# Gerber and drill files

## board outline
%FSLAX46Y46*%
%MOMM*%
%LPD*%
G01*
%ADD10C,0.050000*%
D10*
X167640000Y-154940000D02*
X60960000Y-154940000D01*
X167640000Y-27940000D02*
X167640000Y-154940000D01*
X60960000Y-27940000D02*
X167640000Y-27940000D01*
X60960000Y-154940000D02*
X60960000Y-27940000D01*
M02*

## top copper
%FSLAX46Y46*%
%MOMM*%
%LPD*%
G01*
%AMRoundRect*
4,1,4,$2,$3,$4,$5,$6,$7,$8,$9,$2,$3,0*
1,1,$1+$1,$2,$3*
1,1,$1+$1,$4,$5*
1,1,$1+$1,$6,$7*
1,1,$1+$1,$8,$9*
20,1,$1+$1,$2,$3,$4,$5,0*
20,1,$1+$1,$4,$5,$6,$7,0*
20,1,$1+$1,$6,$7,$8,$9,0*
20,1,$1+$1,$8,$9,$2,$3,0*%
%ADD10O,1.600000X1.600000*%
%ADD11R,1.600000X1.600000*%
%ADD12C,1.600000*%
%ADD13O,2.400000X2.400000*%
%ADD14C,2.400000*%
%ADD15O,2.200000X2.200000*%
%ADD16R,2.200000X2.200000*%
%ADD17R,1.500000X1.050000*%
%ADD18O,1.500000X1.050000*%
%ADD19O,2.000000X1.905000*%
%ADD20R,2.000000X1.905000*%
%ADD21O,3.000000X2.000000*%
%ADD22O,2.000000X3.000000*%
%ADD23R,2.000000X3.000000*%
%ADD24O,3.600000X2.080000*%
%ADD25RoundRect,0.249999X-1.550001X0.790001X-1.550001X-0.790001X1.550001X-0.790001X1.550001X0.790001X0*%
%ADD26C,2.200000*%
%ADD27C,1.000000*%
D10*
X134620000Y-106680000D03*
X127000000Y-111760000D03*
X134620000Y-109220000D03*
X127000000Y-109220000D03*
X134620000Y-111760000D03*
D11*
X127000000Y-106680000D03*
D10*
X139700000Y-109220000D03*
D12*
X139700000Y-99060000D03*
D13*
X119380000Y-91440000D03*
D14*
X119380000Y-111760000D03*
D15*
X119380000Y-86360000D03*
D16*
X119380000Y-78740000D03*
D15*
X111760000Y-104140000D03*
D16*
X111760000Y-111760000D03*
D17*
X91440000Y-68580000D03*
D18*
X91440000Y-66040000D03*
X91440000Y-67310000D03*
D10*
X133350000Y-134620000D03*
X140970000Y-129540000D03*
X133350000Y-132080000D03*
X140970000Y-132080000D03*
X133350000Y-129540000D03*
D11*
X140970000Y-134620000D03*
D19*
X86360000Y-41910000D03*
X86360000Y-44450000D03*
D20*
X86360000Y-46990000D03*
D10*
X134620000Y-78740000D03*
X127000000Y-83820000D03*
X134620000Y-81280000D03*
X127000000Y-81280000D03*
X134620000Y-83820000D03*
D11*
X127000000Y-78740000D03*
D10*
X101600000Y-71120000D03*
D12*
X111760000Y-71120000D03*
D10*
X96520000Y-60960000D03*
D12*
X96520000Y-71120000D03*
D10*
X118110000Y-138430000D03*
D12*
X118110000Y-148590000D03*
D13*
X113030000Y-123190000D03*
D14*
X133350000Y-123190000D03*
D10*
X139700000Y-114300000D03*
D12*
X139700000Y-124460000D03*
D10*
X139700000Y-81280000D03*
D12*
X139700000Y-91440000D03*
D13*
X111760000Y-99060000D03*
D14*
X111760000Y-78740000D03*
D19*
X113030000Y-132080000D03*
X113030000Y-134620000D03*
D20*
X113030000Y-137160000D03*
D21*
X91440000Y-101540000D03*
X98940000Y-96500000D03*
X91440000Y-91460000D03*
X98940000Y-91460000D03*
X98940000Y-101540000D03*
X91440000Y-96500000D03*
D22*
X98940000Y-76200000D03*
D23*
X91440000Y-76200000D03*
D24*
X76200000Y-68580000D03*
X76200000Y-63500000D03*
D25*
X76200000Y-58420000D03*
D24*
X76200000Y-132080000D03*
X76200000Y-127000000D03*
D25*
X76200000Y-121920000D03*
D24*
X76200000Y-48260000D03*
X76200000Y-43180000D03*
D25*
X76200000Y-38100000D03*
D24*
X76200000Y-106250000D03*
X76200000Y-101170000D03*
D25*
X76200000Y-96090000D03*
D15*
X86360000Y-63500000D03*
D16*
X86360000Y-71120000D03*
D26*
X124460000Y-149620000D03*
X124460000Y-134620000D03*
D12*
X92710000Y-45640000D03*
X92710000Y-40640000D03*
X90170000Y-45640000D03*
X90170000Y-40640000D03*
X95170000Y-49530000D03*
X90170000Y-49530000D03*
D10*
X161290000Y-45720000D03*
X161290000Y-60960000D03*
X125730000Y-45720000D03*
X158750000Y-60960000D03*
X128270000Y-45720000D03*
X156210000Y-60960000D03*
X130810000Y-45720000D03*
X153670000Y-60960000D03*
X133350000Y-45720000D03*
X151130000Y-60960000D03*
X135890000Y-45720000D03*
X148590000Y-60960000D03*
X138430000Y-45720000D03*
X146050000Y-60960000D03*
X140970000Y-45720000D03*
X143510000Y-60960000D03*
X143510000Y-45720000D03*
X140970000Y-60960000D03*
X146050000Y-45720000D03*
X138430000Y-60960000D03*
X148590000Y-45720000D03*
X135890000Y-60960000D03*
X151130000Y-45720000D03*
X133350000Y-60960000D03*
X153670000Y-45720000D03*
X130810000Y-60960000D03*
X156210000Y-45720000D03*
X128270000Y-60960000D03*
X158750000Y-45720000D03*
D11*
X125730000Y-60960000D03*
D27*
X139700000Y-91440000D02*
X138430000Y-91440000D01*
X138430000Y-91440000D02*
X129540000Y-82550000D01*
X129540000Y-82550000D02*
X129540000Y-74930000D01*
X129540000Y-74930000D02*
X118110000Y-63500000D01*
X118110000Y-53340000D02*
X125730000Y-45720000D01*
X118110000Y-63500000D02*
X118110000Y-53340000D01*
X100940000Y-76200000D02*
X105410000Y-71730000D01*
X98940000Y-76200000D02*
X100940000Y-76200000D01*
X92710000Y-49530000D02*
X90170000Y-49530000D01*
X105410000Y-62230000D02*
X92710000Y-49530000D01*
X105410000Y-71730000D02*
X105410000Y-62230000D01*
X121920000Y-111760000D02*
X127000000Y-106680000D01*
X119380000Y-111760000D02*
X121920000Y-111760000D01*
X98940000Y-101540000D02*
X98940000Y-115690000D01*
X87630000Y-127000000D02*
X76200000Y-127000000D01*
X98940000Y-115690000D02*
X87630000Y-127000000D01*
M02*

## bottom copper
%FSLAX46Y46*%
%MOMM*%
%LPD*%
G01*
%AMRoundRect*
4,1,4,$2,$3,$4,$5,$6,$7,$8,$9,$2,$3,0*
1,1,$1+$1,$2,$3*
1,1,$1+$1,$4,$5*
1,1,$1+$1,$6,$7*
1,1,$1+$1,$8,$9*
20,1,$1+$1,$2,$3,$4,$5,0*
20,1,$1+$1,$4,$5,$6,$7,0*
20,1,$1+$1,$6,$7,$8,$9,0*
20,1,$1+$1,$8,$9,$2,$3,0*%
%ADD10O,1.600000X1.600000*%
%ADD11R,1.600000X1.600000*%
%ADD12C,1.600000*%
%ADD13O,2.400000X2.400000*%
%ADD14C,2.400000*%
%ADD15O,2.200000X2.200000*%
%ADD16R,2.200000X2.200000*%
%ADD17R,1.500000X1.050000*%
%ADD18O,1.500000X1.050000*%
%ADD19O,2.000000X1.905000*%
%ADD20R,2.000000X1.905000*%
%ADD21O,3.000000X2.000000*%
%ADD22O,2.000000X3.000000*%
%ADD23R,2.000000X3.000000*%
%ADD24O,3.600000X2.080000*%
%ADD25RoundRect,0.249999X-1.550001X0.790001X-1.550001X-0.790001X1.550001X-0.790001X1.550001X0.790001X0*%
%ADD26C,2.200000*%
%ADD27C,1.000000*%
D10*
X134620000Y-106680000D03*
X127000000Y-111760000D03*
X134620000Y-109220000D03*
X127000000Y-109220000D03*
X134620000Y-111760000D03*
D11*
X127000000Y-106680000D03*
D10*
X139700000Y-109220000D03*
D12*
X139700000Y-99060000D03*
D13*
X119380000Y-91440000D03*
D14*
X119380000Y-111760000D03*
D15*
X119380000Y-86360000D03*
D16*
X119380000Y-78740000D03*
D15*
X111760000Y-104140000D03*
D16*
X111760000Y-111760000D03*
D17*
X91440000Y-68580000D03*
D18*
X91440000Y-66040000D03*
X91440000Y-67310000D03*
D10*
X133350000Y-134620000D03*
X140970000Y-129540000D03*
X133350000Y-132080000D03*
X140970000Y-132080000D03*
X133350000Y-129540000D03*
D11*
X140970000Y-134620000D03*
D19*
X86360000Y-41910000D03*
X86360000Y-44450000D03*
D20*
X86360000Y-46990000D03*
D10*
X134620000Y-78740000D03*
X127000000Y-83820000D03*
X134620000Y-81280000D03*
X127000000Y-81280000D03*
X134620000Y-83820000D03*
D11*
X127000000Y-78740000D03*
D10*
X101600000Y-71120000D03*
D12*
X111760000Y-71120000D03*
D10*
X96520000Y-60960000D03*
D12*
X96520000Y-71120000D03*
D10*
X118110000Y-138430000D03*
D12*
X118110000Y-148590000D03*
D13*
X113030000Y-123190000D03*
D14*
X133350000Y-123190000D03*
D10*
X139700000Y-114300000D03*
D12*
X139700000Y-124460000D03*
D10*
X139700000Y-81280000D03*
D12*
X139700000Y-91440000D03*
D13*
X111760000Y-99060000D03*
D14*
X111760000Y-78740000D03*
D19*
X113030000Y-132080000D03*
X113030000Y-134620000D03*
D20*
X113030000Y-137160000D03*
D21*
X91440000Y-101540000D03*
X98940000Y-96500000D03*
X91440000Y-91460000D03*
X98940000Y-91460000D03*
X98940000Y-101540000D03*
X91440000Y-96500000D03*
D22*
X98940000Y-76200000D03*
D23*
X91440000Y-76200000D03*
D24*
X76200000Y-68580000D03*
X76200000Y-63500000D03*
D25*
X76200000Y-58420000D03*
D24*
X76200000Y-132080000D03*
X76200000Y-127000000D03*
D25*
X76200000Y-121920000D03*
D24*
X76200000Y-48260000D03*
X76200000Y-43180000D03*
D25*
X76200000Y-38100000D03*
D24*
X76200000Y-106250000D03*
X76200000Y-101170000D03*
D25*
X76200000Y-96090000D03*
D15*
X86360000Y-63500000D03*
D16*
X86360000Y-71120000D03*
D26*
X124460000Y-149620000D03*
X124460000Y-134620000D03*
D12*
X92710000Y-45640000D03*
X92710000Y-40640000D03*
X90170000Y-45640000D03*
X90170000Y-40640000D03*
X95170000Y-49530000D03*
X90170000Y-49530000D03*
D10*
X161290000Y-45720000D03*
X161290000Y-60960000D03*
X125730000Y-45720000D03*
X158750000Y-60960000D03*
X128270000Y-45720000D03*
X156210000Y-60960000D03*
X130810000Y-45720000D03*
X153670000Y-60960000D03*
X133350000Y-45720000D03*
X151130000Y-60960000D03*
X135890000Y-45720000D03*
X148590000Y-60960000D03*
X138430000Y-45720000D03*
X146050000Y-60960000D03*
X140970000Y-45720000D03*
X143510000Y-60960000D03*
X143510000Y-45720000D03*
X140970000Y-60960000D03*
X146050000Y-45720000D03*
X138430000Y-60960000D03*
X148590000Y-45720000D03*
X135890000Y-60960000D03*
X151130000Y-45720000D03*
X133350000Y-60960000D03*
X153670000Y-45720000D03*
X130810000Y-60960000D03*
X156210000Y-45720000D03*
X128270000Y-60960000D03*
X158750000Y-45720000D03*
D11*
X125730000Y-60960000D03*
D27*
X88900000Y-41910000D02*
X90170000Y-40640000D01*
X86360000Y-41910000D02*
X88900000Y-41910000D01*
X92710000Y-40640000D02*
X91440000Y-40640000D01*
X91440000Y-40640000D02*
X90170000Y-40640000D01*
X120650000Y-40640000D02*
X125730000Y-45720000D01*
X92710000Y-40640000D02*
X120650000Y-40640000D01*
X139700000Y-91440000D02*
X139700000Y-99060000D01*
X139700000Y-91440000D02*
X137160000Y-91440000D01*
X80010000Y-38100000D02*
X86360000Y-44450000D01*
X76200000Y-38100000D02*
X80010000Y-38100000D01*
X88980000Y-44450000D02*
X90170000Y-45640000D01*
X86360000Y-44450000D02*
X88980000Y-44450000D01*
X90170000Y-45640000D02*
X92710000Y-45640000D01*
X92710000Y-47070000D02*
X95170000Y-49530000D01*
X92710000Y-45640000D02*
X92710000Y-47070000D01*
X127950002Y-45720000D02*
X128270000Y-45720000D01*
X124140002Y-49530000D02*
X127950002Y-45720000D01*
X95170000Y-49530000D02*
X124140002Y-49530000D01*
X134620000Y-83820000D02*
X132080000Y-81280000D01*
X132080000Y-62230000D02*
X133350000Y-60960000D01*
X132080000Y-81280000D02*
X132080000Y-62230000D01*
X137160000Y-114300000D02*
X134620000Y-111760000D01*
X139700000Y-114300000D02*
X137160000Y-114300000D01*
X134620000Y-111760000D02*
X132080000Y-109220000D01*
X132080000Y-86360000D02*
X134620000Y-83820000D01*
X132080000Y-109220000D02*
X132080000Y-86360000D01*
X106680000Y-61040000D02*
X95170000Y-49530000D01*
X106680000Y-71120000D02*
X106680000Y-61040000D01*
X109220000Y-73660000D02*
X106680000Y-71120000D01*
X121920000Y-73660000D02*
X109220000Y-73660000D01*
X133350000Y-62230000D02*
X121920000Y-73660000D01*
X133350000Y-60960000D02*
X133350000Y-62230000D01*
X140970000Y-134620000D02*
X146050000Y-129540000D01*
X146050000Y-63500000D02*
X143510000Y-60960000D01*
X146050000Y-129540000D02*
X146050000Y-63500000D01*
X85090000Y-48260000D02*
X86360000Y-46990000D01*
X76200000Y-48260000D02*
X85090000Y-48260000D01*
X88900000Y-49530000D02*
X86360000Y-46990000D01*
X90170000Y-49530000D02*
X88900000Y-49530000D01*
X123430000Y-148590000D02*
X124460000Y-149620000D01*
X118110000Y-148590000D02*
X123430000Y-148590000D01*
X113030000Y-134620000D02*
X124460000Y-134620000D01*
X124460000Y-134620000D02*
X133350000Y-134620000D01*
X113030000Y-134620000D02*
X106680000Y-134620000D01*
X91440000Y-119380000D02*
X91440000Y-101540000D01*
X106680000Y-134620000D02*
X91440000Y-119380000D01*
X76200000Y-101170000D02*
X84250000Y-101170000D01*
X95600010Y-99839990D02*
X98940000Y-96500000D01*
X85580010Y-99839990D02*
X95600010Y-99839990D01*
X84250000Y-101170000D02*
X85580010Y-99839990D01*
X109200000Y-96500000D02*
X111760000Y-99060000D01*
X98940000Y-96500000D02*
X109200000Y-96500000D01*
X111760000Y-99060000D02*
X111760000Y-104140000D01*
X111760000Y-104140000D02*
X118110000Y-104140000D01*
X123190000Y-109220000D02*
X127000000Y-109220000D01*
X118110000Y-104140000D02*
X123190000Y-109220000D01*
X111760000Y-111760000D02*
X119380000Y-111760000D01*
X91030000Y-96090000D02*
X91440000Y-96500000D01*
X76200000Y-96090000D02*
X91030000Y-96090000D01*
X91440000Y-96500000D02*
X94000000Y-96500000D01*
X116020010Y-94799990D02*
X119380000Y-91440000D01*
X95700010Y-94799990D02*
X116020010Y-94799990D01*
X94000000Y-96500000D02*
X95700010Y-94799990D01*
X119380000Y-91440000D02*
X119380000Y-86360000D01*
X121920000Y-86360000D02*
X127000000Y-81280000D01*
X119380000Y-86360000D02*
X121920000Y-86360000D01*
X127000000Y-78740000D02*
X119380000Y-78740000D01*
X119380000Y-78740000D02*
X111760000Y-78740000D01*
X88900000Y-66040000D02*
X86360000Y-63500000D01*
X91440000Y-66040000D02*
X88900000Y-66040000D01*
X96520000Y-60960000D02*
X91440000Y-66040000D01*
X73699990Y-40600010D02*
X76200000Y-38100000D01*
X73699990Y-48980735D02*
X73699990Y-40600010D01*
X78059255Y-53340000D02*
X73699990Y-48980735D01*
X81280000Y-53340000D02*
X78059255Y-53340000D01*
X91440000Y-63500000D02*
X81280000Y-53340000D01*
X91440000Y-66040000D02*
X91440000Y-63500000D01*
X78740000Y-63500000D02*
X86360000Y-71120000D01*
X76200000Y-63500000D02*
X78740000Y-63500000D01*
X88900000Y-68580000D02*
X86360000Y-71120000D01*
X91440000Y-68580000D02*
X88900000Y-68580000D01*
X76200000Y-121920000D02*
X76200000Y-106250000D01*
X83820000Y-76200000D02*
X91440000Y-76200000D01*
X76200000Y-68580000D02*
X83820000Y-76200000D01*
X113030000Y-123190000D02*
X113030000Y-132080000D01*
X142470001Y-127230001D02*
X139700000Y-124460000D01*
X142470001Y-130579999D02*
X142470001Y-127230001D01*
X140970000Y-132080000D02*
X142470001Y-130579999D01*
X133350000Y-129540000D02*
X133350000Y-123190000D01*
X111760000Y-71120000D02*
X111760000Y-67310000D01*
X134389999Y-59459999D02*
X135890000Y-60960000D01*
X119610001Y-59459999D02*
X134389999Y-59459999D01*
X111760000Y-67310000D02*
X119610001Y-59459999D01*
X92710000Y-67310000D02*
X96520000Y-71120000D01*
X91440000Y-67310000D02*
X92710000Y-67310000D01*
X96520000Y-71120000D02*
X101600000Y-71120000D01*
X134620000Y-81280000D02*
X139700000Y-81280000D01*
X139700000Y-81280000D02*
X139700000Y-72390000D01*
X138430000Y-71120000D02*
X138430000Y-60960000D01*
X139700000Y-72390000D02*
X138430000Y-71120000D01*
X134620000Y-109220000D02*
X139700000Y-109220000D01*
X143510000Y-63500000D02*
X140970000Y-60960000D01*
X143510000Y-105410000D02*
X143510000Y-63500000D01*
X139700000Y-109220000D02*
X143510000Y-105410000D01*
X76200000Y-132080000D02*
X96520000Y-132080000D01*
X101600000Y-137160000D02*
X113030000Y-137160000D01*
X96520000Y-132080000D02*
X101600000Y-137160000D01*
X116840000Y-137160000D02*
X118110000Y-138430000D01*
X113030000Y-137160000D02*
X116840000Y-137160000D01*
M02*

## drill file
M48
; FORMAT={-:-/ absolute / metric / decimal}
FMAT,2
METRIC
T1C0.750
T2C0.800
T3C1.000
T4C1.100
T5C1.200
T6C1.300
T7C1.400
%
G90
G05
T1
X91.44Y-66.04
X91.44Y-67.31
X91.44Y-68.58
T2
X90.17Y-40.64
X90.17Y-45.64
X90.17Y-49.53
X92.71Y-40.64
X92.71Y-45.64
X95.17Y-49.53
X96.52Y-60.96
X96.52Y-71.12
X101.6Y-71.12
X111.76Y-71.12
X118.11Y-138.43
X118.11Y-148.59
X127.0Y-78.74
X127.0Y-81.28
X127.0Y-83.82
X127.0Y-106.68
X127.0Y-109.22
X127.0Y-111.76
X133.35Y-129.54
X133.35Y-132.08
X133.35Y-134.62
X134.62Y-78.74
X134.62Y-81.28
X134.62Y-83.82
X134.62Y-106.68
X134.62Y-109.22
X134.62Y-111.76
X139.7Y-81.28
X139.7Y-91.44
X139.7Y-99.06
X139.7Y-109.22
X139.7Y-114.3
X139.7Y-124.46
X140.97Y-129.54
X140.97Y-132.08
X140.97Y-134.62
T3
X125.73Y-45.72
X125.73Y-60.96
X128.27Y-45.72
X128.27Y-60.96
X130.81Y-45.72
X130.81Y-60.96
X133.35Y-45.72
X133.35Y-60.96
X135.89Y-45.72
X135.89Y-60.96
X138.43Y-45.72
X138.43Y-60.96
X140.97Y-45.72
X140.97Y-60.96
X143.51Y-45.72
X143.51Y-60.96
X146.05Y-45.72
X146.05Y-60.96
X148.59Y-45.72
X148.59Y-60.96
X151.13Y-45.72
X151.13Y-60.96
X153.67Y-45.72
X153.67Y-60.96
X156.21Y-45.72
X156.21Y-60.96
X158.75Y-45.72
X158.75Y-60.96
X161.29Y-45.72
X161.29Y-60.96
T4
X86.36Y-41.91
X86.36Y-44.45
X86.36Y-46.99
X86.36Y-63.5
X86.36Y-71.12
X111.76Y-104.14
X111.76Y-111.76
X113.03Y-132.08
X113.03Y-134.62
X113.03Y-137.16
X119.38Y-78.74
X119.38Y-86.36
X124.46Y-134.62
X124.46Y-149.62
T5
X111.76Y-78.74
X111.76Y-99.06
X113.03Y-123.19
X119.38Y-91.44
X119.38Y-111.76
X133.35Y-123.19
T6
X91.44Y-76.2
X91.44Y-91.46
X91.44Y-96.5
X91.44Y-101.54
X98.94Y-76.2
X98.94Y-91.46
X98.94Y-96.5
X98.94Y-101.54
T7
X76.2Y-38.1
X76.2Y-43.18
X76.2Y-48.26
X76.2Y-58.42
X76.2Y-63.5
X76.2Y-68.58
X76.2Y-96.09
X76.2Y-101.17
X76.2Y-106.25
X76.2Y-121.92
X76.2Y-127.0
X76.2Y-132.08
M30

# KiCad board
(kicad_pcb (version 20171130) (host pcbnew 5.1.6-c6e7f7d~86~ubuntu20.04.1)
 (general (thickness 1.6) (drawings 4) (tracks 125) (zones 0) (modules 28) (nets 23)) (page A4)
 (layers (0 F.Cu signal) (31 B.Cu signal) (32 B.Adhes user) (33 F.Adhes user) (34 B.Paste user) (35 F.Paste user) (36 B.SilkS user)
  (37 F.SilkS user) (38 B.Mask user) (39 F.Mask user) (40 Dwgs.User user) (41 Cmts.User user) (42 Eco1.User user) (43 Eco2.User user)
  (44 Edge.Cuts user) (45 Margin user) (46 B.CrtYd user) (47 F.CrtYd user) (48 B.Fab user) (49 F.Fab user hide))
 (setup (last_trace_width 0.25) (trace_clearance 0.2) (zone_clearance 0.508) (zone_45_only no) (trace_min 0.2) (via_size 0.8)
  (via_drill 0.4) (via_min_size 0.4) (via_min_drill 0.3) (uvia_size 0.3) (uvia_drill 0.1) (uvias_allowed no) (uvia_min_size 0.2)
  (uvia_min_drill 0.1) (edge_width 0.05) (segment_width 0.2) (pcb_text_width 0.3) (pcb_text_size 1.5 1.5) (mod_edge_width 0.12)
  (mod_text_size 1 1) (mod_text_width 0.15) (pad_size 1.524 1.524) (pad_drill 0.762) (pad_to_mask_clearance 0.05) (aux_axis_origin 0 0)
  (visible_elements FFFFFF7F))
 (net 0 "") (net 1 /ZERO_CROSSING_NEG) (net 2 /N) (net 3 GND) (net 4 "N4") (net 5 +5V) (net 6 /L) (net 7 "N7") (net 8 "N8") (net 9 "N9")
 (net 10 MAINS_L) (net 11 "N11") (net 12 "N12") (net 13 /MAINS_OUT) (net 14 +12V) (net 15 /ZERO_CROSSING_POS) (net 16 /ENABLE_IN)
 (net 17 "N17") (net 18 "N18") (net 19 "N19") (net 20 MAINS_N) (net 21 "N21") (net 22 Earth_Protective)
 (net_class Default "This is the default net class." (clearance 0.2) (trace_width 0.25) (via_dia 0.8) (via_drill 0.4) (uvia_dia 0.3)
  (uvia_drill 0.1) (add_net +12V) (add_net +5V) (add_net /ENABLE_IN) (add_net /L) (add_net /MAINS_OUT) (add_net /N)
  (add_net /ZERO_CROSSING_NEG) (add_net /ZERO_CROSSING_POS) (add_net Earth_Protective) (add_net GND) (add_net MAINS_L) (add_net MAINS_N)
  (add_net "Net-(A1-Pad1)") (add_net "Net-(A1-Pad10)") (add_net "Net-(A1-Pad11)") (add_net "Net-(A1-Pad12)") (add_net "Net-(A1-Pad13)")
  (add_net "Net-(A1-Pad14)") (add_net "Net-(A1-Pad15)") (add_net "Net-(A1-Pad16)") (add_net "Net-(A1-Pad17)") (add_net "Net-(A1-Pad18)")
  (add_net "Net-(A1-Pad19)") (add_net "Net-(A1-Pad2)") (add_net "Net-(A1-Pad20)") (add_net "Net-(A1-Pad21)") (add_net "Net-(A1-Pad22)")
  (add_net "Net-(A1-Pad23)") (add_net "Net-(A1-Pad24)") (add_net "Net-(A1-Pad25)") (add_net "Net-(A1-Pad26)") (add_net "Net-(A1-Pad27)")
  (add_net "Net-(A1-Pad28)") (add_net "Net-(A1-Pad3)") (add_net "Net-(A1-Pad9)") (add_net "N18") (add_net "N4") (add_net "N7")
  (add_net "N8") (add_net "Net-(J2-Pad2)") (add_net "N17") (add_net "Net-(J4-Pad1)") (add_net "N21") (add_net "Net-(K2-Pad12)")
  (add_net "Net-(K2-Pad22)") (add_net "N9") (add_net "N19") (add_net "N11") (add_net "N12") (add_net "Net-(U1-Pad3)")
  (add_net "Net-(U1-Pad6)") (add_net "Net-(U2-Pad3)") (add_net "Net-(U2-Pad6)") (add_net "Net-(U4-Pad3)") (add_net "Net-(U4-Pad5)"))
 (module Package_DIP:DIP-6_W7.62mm (layer F.Cu) (at 127 106.68)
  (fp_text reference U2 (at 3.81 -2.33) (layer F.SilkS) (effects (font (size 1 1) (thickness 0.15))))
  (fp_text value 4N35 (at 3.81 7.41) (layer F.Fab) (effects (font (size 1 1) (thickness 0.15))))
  (pad 6 thru_hole oval (at 7.62 0) (size 1.6 1.6) (drill 0.8) (layers *.Cu *.Mask))
  (pad 3 thru_hole oval (at 0 5.08) (size 1.6 1.6) (drill 0.8) (layers *.Cu *.Mask))
  (pad 5 thru_hole oval (at 7.62 2.54) (size 1.6 1.6) (drill 0.8) (layers *.Cu *.Mask) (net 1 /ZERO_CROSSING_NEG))
  (pad 2 thru_hole oval (at 0 2.54) (size 1.6 1.6) (drill 0.8) (layers *.Cu *.Mask) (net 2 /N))
  (pad 4 thru_hole oval (at 7.62 5.08) (size 1.6 1.6) (drill 0.8) (layers *.Cu *.Mask) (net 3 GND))
  (pad 1 thru_hole rect (at 0 0) (size 1.6 1.6) (drill 0.8) (layers *.Cu *.Mask) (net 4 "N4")))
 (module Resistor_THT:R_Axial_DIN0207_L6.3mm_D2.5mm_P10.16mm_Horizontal (layer F.Cu) (at 139.7 99.06 270)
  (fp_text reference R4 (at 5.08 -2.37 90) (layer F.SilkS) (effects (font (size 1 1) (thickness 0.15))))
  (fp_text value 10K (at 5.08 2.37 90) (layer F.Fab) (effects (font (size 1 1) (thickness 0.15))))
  (pad 2 thru_hole oval (at 10.16 0 270) (size 1.6 1.6) (drill 0.8) (layers *.Cu *.Mask) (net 1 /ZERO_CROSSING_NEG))
  (pad 1 thru_hole circle (at 0 0 270) (size 1.6 1.6) (drill 0.8) (layers *.Cu *.Mask) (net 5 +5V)))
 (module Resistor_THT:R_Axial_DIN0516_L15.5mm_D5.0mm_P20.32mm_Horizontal (layer F.Cu) (at 119.38 111.76 90)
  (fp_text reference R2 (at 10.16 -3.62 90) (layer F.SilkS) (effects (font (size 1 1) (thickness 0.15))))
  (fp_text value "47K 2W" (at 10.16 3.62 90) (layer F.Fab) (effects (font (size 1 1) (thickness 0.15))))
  (pad 2 thru_hole oval (at 20.32 0 90) (size 2.4 2.4) (drill 1.2) (layers *.Cu *.Mask) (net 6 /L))
  (pad 1 thru_hole circle (at 0 0 90) (size 2.4 2.4) (drill 1.2) (layers *.Cu *.Mask) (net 4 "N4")))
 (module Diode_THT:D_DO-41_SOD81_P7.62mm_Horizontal (layer F.Cu) (at 119.38 78.74 270)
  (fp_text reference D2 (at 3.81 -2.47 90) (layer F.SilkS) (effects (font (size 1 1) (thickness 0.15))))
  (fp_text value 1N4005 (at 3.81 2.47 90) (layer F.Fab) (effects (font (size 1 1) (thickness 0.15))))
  (pad 2 thru_hole oval (at 7.62 0 270) (size 2.2 2.2) (drill 1.1) (layers *.Cu *.Mask) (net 6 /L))
  (pad 1 thru_hole rect (at 0 0 270) (size 2.2 2.2) (drill 1.1) (layers *.Cu *.Mask) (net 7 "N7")))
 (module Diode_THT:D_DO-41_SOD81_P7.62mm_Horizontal (layer F.Cu) (at 111.76 111.76 90)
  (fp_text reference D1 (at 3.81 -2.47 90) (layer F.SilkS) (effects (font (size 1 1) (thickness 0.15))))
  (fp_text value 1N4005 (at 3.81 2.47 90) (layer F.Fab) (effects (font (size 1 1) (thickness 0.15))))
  (pad 2 thru_hole oval (at 7.62 0 90) (size 2.2 2.2) (drill 1.1) (layers *.Cu *.Mask) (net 2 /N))
  (pad 1 thru_hole rect (at 0 0 90) (size 2.2 2.2) (drill 1.1) (layers *.Cu *.Mask) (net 4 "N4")))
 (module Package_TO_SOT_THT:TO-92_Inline (layer F.Cu) (at 91.44 68.58 90)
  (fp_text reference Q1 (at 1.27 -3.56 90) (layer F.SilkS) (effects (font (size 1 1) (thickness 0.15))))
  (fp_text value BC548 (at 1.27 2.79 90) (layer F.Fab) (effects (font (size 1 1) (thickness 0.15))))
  (pad 1 thru_hole rect (at 0 0 90) (size 1.05 1.5) (drill 0.75) (layers *.Cu *.Mask) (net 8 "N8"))
  (pad 3 thru_hole oval (at 2.54 0 90) (size 1.05 1.5) (drill 0.75) (layers *.Cu *.Mask) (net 3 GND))
  (pad 2 thru_hole oval (at 1.27 0 90) (size 1.05 1.5) (drill 0.75) (layers *.Cu *.Mask) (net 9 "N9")))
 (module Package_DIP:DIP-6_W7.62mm (layer F.Cu) (at 140.97 134.62 180)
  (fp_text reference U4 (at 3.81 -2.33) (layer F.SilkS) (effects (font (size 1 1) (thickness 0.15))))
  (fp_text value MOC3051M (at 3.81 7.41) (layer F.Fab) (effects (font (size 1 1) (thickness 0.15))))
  (pad 6 thru_hole oval (at 7.62 0 180) (size 1.6 1.6) (drill 0.8) (layers *.Cu *.Mask) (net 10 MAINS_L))
  (pad 3 thru_hole oval (at 0 5.08 180) (size 1.6 1.6) (drill 0.8) (layers *.Cu *.Mask))
  (pad 5 thru_hole oval (at 7.62 2.54 180) (size 1.6 1.6) (drill 0.8) (layers *.Cu *.Mask))
  (pad 2 thru_hole oval (at 0 2.54 180) (size 1.6 1.6) (drill 0.8) (layers *.Cu *.Mask) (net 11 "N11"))
  (pad 4 thru_hole oval (at 7.62 5.08 180) (size 1.6 1.6) (drill 0.8) (layers *.Cu *.Mask) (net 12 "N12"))
  (pad 1 thru_hole rect (at 0 0 180) (size 1.6 1.6) (drill 0.8) (layers *.Cu *.Mask) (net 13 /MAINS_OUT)))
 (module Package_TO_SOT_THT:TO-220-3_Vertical (layer F.Cu) (at 86.36 46.99 90)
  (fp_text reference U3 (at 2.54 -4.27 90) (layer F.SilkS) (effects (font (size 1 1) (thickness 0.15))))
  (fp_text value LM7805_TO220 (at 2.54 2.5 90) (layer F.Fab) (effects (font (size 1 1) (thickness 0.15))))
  (pad 3 thru_hole oval (at 5.08 0 90) (size 1.905 2) (drill 1.1) (layers *.Cu *.Mask) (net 5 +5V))
  (pad 2 thru_hole oval (at 2.54 0 90) (size 1.905 2) (drill 1.1) (layers *.Cu *.Mask) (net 3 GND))
  (pad 1 thru_hole rect (at 0 0 90) (size 1.905 2) (drill 1.1) (layers *.Cu *.Mask) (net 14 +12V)))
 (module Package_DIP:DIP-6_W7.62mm (layer F.Cu) (at 127 78.74)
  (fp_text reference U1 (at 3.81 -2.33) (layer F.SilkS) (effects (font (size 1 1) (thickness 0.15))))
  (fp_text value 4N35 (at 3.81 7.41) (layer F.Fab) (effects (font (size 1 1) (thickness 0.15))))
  (pad 6 thru_hole oval (at 7.62 0) (size 1.6 1.6) (drill 0.8) (layers *.Cu *.Mask))
  (pad 3 thru_hole oval (at 0 5.08) (size 1.6 1.6) (drill 0.8) (layers *.Cu *.Mask))
  (pad 5 thru_hole oval (at 7.62 2.54) (size 1.6 1.6) (drill 0.8) (layers *.Cu *.Mask) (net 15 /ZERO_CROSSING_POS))
  (pad 2 thru_hole oval (at 0 2.54) (size 1.6 1.6) (drill 0.8) (layers *.Cu *.Mask) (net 6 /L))
  (pad 4 thru_hole oval (at 7.62 5.08) (size 1.6 1.6) (drill 0.8) (layers *.Cu *.Mask) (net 3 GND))
  (pad 1 thru_hole rect (at 0 0) (size 1.6 1.6) (drill 0.8) (layers *.Cu *.Mask) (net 7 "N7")))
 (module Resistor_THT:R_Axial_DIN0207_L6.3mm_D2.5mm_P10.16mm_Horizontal (layer F.Cu) (at 111.76 71.12 180)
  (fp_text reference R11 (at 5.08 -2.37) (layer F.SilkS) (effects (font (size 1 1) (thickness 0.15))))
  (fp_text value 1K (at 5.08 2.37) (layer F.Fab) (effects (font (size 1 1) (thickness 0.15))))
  (pad 2 thru_hole oval (at 10.16 0 180) (size 1.6 1.6) (drill 0.8) (layers *.Cu *.Mask) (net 9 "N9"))
  (pad 1 thru_hole circle (at 0 0 180) (size 1.6 1.6) (drill 0.8) (layers *.Cu *.Mask) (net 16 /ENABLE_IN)))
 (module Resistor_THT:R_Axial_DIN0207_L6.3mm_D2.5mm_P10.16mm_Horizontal (layer F.Cu) (at 96.52 71.12 90)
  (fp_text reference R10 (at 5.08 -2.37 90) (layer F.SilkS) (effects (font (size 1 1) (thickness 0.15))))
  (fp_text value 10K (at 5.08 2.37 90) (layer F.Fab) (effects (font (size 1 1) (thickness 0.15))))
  (pad 2 thru_hole oval (at 10.16 0 90) (size 1.6 1.6) (drill 0.8) (layers *.Cu *.Mask) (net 3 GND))
  (pad 1 thru_hole circle (at 0 0 90) (size 1.6 1.6) (drill 0.8) (layers *.Cu *.Mask) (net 9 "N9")))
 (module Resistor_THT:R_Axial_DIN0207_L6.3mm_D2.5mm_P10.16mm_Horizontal (layer F.Cu) (at 118.11 148.59 90)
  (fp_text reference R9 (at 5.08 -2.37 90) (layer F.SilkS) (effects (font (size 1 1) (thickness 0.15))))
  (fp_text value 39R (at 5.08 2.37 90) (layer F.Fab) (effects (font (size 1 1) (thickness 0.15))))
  (pad 2 thru_hole oval (at 10.16 0 90) (size 1.6 1.6) (drill 0.8) (layers *.Cu *.Mask) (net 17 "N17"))
  (pad 1 thru_hole circle (at 0 0 90) (size 1.6 1.6) (drill 0.8) (layers *.Cu *.Mask) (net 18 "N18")))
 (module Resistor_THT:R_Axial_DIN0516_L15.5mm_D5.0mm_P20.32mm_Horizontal (layer F.Cu) (at 133.35 123.19 180)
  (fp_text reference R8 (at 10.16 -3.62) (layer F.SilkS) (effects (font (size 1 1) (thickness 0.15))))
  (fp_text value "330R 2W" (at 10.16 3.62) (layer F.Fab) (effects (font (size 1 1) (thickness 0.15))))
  (pad 2 thru_hole oval (at 20.32 0 180) (size 2.4 2.4) (drill 1.2) (layers *.Cu *.Mask) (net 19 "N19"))
  (pad 1 thru_hole circle (at 0 0 180) (size 2.4 2.4) (drill 1.2) (layers *.Cu *.Mask) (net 12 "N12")))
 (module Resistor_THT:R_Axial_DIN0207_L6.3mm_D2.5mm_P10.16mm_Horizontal (layer F.Cu) (at 139.7 124.46 90)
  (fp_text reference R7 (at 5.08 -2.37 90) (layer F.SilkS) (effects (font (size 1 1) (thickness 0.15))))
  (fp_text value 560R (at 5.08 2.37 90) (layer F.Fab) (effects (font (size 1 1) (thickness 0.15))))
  (pad 2 thru_hole oval (at 10.16 0 90) (size 1.6 1.6) (drill 0.8) (layers *.Cu *.Mask) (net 3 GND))
  (pad 1 thru_hole circle (at 0 0 90) (size 1.6 1.6) (drill 0.8) (layers *.Cu *.Mask) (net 11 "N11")))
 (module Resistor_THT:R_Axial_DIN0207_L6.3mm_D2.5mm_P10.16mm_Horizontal (layer F.Cu) (at 139.7 91.44 90)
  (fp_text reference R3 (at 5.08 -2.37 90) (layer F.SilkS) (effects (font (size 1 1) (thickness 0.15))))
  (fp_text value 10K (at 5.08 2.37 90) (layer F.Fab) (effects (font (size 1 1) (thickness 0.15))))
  (pad 2 thru_hole oval (at 10.16 0 90) (size 1.6 1.6) (drill 0.8) (layers *.Cu *.Mask) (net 15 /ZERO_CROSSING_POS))
  (pad 1 thru_hole circle (at 0 0 90) (size 1.6 1.6) (drill 0.8) (layers *.Cu *.Mask) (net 5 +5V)))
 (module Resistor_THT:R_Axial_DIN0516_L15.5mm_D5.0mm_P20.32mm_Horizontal (layer F.Cu) (at 111.76 78.74 270)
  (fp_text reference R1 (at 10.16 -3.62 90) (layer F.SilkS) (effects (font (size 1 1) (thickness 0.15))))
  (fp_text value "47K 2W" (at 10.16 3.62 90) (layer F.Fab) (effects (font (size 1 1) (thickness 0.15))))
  (pad 2 thru_hole oval (at 20.32 0 270) (size 2.4 2.4) (drill 1.2) (layers *.Cu *.Mask) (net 2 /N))
  (pad 1 thru_hole circle (at 0 0 270) (size 2.4 2.4) (drill 1.2) (layers *.Cu *.Mask) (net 7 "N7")))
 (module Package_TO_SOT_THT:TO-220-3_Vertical (layer F.Cu) (at 113.03 137.16 90)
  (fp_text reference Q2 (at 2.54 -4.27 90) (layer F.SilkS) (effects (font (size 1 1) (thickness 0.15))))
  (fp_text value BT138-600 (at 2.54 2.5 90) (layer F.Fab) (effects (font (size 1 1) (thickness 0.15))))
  (pad 3 thru_hole oval (at 5.08 0 90) (size 1.905 2) (drill 1.1) (layers *.Cu *.Mask) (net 19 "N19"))
  (pad 2 thru_hole oval (at 2.54 0 90) (size 1.905 2) (drill 1.1) (layers *.Cu *.Mask) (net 10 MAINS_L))
  (pad 1 thru_hole rect (at 0 0 90) (size 1.905 2) (drill 1.1) (layers *.Cu *.Mask) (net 17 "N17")))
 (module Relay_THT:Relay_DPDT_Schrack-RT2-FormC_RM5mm (layer F.Cu) (at 91.44 76.2 270)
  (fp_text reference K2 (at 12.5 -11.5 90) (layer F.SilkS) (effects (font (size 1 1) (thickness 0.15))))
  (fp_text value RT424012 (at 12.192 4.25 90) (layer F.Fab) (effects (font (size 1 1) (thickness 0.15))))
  (pad 14 thru_hole oval (at 25.34 0 90) (size 2 3) (drill 1.3) (layers *.Cu *.Mask) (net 10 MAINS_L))
  (pad 21 thru_hole oval (at 20.3 -7.5 90) (size 2 3) (drill 1.3) (layers *.Cu *.Mask) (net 2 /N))
  (pad 12 thru_hole oval (at 15.26 0 90) (size 2 3) (drill 1.3) (layers *.Cu *.Mask))
  (pad 22 thru_hole oval (at 15.26 -7.5 90) (size 2 3) (drill 1.3) (layers *.Cu *.Mask))
  (pad 24 thru_hole oval (at 25.34 -7.5 90) (size 2 3) (drill 1.3) (layers *.Cu *.Mask) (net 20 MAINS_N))
  (pad 11 thru_hole oval (at 20.3 0 90) (size 2 3) (drill 1.3) (layers *.Cu *.Mask) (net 6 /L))
  (pad A2 thru_hole oval (at 0 -7.5 90) (size 3 2) (drill 1.3) (layers *.Cu *.Mask) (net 14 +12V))
  (pad A1 thru_hole rect (at 0 0 90) (size 3 2) (drill 1.3) (layers *.Cu *.Mask) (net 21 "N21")))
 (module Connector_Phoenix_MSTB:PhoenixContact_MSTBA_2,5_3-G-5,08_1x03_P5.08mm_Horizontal (layer F.Cu) (at 76.2 58.42 270)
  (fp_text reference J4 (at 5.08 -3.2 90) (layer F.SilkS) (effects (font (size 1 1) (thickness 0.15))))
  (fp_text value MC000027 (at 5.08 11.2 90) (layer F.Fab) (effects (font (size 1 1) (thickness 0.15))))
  (pad 3 thru_hole oval (at 10.16 0 270) (size 2.08 3.6) (drill 1.4) (layers *.Cu *.Mask) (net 21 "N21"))
  (pad 2 thru_hole oval (at 5.08 0 270) (size 2.08 3.6) (drill 1.4) (layers *.Cu *.Mask) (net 8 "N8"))
  (pad 1 thru_hole roundrect (at 0 0 270) (size 2.08 3.6) (drill 1.4) (layers *.Cu *.Mask) (roundrect_rratio 0.120192)))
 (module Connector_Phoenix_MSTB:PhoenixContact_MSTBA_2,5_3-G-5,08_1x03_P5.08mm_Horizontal (layer F.Cu) (at 76.2 121.92 270)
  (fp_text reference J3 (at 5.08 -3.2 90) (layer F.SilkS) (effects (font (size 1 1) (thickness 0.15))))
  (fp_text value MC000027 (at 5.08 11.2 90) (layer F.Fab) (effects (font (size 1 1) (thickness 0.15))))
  (pad 3 thru_hole oval (at 10.16 0 270) (size 2.08 3.6) (drill 1.4) (layers *.Cu *.Mask) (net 17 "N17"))
  (pad 2 thru_hole oval (at 5.08 0 270) (size 2.08 3.6) (drill 1.4) (layers *.Cu *.Mask) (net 20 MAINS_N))
  (pad 1 thru_hole roundrect (at 0 0 270) (size 2.08 3.6) (drill 1.4) (layers *.Cu *.Mask) (roundrect_rratio 0.120192)
   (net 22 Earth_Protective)))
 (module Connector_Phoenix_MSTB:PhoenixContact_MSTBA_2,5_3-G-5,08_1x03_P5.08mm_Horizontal (layer F.Cu) (at 76.2 38.1 270)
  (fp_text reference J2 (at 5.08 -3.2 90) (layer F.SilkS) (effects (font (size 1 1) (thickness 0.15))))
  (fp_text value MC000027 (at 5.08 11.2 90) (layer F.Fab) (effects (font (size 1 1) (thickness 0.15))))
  (pad 3 thru_hole oval (at 10.16 0 270) (size 2.08 3.6) (drill 1.4) (layers *.Cu *.Mask) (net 14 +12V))
  (pad 2 thru_hole oval (at 5.08 0 270) (size 2.08 3.6) (drill 1.4) (layers *.Cu *.Mask))
  (pad 1 thru_hole roundrect (at 0 0 270) (size 2.08 3.6) (drill 1.4) (layers *.Cu *.Mask) (roundrect_rratio 0.120192) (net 3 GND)))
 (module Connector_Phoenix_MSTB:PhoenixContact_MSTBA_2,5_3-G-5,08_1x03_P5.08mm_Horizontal (layer F.Cu) (at 76.2 96.09 270)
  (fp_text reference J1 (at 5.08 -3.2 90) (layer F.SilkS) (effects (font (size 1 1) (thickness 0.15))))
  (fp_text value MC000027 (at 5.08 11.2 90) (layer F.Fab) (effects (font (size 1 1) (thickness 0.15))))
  (pad 3 thru_hole oval (at 10.16 0 270) (size 2.08 3.6) (drill 1.4) (layers *.Cu *.Mask) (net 22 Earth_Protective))
  (pad 2 thru_hole oval (at 5.08 0 270) (size 2.08 3.6) (drill 1.4) (layers *.Cu *.Mask) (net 2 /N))
  (pad 1 thru_hole roundrect (at 0 0 270) (size 2.08 3.6) (drill 1.4) (layers *.Cu *.Mask) (roundrect_rratio 0.120192) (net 6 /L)))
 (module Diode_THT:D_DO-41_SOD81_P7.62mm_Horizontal (layer F.Cu) (at 86.36 71.12 90)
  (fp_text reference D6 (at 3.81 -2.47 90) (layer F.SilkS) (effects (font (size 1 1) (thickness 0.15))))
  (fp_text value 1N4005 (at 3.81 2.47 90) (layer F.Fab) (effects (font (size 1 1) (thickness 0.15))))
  (pad 2 thru_hole oval (at 7.62 0 90) (size 2.2 2.2) (drill 1.1) (layers *.Cu *.Mask) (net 3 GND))
  (pad 1 thru_hole rect (at 0 0 90) (size 2.2 2.2) (drill 1.1) (layers *.Cu *.Mask) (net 8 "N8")))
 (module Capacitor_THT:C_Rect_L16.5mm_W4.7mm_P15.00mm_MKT (layer F.Cu) (at 124.46 134.62 270)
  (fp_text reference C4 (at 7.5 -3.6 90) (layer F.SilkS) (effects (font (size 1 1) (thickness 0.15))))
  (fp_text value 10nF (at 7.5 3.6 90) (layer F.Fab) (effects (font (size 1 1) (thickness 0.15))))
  (pad 2 thru_hole circle (at 15 0 270) (size 2.2 2.2) (drill 1.1) (layers *.Cu *.Mask) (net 18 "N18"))
  (pad 1 thru_hole circle (at 0 0 270) (size 2.2 2.2) (drill 1.1) (layers *.Cu *.Mask) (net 10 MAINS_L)))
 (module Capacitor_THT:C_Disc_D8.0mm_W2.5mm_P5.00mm (layer F.Cu) (at 92.71 40.64 270)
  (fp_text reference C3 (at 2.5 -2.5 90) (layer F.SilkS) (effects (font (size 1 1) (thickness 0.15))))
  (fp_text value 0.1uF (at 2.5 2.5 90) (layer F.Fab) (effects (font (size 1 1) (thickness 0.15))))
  (pad 2 thru_hole circle (at 5 0 270) (size 1.6 1.6) (drill 0.8) (layers *.Cu *.Mask) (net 3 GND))
  (pad 1 thru_hole circle (at 0 0 270) (size 1.6 1.6) (drill 0.8) (layers *.Cu *.Mask) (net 5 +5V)))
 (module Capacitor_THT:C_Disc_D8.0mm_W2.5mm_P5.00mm (layer F.Cu) (at 90.17 40.64 270)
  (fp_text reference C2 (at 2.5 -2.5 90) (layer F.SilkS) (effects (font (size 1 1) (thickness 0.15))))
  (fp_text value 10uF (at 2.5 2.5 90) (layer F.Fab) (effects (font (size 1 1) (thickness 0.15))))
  (pad 2 thru_hole circle (at 5 0 270) (size 1.6 1.6) (drill 0.8) (layers *.Cu *.Mask) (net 3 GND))
  (pad 1 thru_hole circle (at 0 0 270) (size 1.6 1.6) (drill 0.8) (layers *.Cu *.Mask) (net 5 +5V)))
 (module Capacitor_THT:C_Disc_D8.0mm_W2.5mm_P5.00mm (layer F.Cu) (at 90.17 49.53)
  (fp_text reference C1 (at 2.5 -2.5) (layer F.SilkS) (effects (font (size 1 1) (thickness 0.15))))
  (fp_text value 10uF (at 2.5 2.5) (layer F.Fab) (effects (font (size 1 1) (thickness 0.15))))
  (pad 2 thru_hole circle (at 5 0) (size 1.6 1.6) (drill 0.8) (layers *.Cu *.Mask) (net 3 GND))
  (pad 1 thru_hole circle (at 0 0) (size 1.6 1.6) (drill 0.8) (layers *.Cu *.Mask) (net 14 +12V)))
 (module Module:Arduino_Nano (layer F.Cu) (at 125.73 60.96 90)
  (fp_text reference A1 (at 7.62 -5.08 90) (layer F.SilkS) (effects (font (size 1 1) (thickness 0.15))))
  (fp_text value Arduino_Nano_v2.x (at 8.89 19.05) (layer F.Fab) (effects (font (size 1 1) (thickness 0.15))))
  (pad 16 thru_hole oval (at 15.24 35.56 90) (size 1.6 1.6) (drill 1) (layers *.Cu *.Mask))
  (pad 15 thru_hole oval (at 0 35.56 90) (size 1.6 1.6) (drill 1) (layers *.Cu *.Mask))
  (pad 30 thru_hole oval (at 15.24 0 90) (size 1.6 1.6) (drill 1) (layers *.Cu *.Mask) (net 5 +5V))
  (pad 14 thru_hole oval (at 0 33.02 90) (size 1.6 1.6) (drill 1) (layers *.Cu *.Mask))
  (pad 29 thru_hole oval (at 15.24 2.54 90) (size 1.6 1.6) (drill 1) (layers *.Cu *.Mask) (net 3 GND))
  (pad 13 thru_hole oval (at 0 30.48 90) (size 1.6 1.6) (drill 1) (layers *.Cu *.Mask))
  (pad 28 thru_hole oval (at 15.24 5.08 90) (size 1.6 1.6) (drill 1) (layers *.Cu *.Mask))
  (pad 12 thru_hole oval (at 0 27.94 90) (size 1.6 1.6) (drill 1) (layers *.Cu *.Mask))
  (pad 27 thru_hole oval (at 15.24 7.62 90) (size 1.6 1.6) (drill 1) (layers *.Cu *.Mask))
  (pad 11 thru_hole oval (at 0 25.4 90) (size 1.6 1.6) (drill 1) (layers *.Cu *.Mask))
  (pad 26 thru_hole oval (at 15.24 10.16 90) (size 1.6 1.6) (drill 1) (layers *.Cu *.Mask))
  (pad 10 thru_hole oval (at 0 22.86 90) (size 1.6 1.6) (drill 1) (layers *.Cu *.Mask))
  (pad 25 thru_hole oval (at 15.24 12.7 90) (size 1.6 1.6) (drill 1) (layers *.Cu *.Mask))
  (pad 9 thru_hole oval (at 0 20.32 90) (size 1.6 1.6) (drill 1) (layers *.Cu *.Mask))
  (pad 24 thru_hole oval (at 15.24 15.24 90) (size 1.6 1.6) (drill 1) (layers *.Cu *.Mask))
  (pad 8 thru_hole oval (at 0 17.78 90) (size 1.6 1.6) (drill 1) (layers *.Cu *.Mask) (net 13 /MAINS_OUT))
  (pad 23 thru_hole oval (at 15.24 17.78 90) (size 1.6 1.6) (drill 1) (layers *.Cu *.Mask))
  (pad 7 thru_hole oval (at 0 15.24 90) (size 1.6 1.6) (drill 1) (layers *.Cu *.Mask) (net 1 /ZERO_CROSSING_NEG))
  (pad 22 thru_hole oval (at 15.24 20.32 90) (size 1.6 1.6) (drill 1) (layers *.Cu *.Mask))
  (pad 6 thru_hole oval (at 0 12.7 90) (size 1.6 1.6) (drill 1) (layers *.Cu *.Mask) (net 15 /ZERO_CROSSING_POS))
  (pad 21 thru_hole oval (at 15.24 22.86 90) (size 1.6 1.6) (drill 1) (layers *.Cu *.Mask))
  (pad 5 thru_hole oval (at 0 10.16 90) (size 1.6 1.6) (drill 1) (layers *.Cu *.Mask) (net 16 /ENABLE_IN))
  (pad 20 thru_hole oval (at 15.24 25.4 90) (size 1.6 1.6) (drill 1) (layers *.Cu *.Mask))
  (pad 4 thru_hole oval (at 0 7.62 90) (size 1.6 1.6) (drill 1) (layers *.Cu *.Mask) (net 3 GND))
  (pad 19 thru_hole oval (at 15.24 27.94 90) (size 1.6 1.6) (drill 1) (layers *.Cu *.Mask))
  (pad 3 thru_hole oval (at 0 5.08 90) (size 1.6 1.6) (drill 1) (layers *.Cu *.Mask))
  (pad 18 thru_hole oval (at 15.24 30.48 90) (size 1.6 1.6) (drill 1) (layers *.Cu *.Mask))
  (pad 2 thru_hole oval (at 0 2.54 90) (size 1.6 1.6) (drill 1) (layers *.Cu *.Mask))
  (pad 17 thru_hole oval (at 15.24 33.02 90) (size 1.6 1.6) (drill 1) (layers *.Cu *.Mask))
  (pad 1 thru_hole rect (at 0 0 90) (size 1.6 1.6) (drill 1) (layers *.Cu *.Mask)))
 (gr_line (start 167.64 154.94) (end 60.96 154.94) (layer Edge.Cuts) (width 0.05))
 (gr_line (start 167.64 27.94) (end 167.64 154.94) (layer Edge.Cuts) (width 0.05))
 (gr_line (start 60.96 27.94) (end 167.64 27.94) (layer Edge.Cuts) (width 0.05))
 (gr_line (start 60.96 154.94) (end 60.96 27.94) (layer Edge.Cuts) (width 0.05))
 (segment (start 88.9 41.91) (end 90.17 40.64) (width 1) (layer B.Cu) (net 5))
 (segment (start 86.36 41.91) (end 88.9 41.91) (width 1) (layer B.Cu) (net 5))
 (segment (start 92.71 40.64) (end 91.44 40.64) (width 1) (layer B.Cu) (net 5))
 (segment (start 91.44 40.64) (end 90.17 40.64) (width 1) (layer B.Cu) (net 5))
 (segment (start 120.65 40.64) (end 125.73 45.72) (width 1) (layer B.Cu) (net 5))
 (segment (start 92.71 40.64) (end 120.65 40.64) (width 1) (layer B.Cu) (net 5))
 (segment (start 139.7 91.44) (end 139.7 99.06) (width 1) (layer B.Cu) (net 5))
 (segment (start 139.7 91.44) (end 137.16 91.44) (width 1) (layer B.Cu) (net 5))
 (segment (start 139.7 91.44) (end 138.43 91.44) (width 1) (layer F.Cu) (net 5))
 (segment (start 138.43 91.44) (end 129.54 82.55) (width 1) (layer F.Cu) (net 5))
 (segment (start 129.54 82.55) (end 129.54 74.93) (width 1) (layer F.Cu) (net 5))
 (segment (start 129.54 74.93) (end 118.11 63.5) (width 1) (layer F.Cu) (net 5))
 (segment (start 118.11 53.34) (end 125.73 45.72) (width 1) (layer F.Cu) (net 5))
 (segment (start 118.11 63.5) (end 118.11 53.34) (width 1) (layer F.Cu) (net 5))
 (segment (start 80.01 38.1) (end 86.36 44.45) (width 1) (layer B.Cu) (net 3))
 (segment (start 76.2 38.1) (end 80.01 38.1) (width 1) (layer B.Cu) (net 3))
 (segment (start 88.98 44.45) (end 90.17 45.64) (width 1) (layer B.Cu) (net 3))
 (segment (start 86.36 44.45) (end 88.98 44.45) (width 1) (layer B.Cu) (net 3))
 (segment (start 90.17 45.64) (end 92.71 45.64) (width 1) (layer B.Cu) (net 3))
 (segment (start 92.71 47.07) (end 95.17 49.53) (width 1) (layer B.Cu) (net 3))
 (segment (start 92.71 45.64) (end 92.71 47.07) (width 1) (layer B.Cu) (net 3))
 (segment (start 127.950002 45.72) (end 128.27 45.72) (width 1) (layer B.Cu) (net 3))
 (segment (start 124.140002 49.53) (end 127.950002 45.72) (width 1) (layer B.Cu) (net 3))
 (segment (start 95.17 49.53) (end 124.140002 49.53) (width 1) (layer B.Cu) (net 3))
 (segment (start 134.62 83.82) (end 132.08 81.28) (width 1) (layer B.Cu) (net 3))
 (segment (start 132.08 62.23) (end 133.35 60.96) (width 1) (layer B.Cu) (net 3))
 (segment (start 132.08 81.28) (end 132.08 62.23) (width 1) (layer B.Cu) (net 3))
 (segment (start 137.16 114.3) (end 134.62 111.76) (width 1) (layer B.Cu) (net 3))
 (segment (start 139.7 114.3) (end 137.16 114.3) (width 1) (layer B.Cu) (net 3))
 (segment (start 134.62 111.76) (end 132.08 109.22) (width 1) (layer B.Cu) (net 3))
 (segment (start 132.08 86.36) (end 134.62 83.82) (width 1) (layer B.Cu) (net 3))
 (segment (start 132.08 109.22) (end 132.08 86.36) (width 1) (layer B.Cu) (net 3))
 (segment (start 106.68 61.04) (end 95.17 49.53) (width 1) (layer B.Cu) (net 3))
 (segment (start 106.68 71.12) (end 106.68 61.04) (width 1) (layer B.Cu) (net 3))
 (segment (start 109.22 73.66) (end 106.68 71.12) (width 1) (layer B.Cu) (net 3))
 (segment (start 121.92 73.66) (end 109.22 73.66) (width 1) (layer B.Cu) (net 3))
 (segment (start 133.35 62.23) (end 121.92 73.66) (width 1) (layer B.Cu) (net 3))
 (segment (start 133.35 60.96) (end 133.35 62.23) (width 1) (layer B.Cu) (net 3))
 (segment (start 140.97 134.62) (end 146.05 129.54) (width 1) (layer B.Cu) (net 13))
 (segment (start 146.05 63.5) (end 143.51 60.96) (width 1) (layer B.Cu) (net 13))
 (segment (start 146.05 129.54) (end 146.05 63.5) (width 1) (layer B.Cu) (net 13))
 (segment (start 85.09 48.26) (end 86.36 46.99) (width 1) (layer B.Cu) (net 14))
 (segment (start 76.2 48.26) (end 85.09 48.26) (width 1) (layer B.Cu) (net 14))
 (segment (start 88.9 49.53) (end 86.36 46.99) (width 1) (layer B.Cu) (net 14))
 (segment (start 90.17 49.53) (end 88.9 49.53) (width 1) (layer B.Cu) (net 14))
 (segment (start 100.94 76.2) (end 105.41 71.73) (width 1) (layer F.Cu) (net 14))
 (segment (start 98.94 76.2) (end 100.94 76.2) (width 1) (layer F.Cu) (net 14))
 (segment (start 92.71 49.53) (end 90.17 49.53) (width 1) (layer F.Cu) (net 14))
 (segment (start 105.41 62.23) (end 92.71 49.53) (width 1) (layer F.Cu) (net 14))
 (segment (start 105.41 71.73) (end 105.41 62.23) (width 1) (layer F.Cu) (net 14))
 (segment (start 123.43 148.59) (end 124.46 149.62) (width 1) (layer B.Cu) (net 18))
 (segment (start 118.11 148.59) (end 123.43 148.59) (width 1) (layer B.Cu) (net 18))
 (segment (start 113.03 134.62) (end 124.46 134.62) (width 1) (layer B.Cu) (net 10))
 (segment (start 124.46 134.62) (end 133.35 134.62) (width 1) (layer B.Cu) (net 10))
 (segment (start 113.03 134.62) (end 106.68 134.62) (width 1) (layer B.Cu) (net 10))
 (segment (start 91.44 119.38) (end 91.44 101.54) (width 1) (layer B.Cu) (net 10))
 (segment (start 106.68 134.62) (end 91.44 119.38) (width 1) (layer B.Cu) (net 10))
 (segment (start 76.2 101.17) (end 84.25 101.17) (width 1) (layer B.Cu) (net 2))
 (segment (start 95.60001 99.83999) (end 98.94 96.5) (width 1) (layer B.Cu) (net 2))
 (segment (start 85.58001 99.83999) (end 95.60001 99.83999) (width 1) (layer B.Cu) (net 2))
 (segment (start 84.25 101.17) (end 85.58001 99.83999) (width 1) (layer B.Cu) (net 2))
 (segment (start 109.2 96.5) (end 111.76 99.06) (width 1) (layer B.Cu) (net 2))
 (segment (start 98.94 96.5) (end 109.2 96.5) (width 1) (layer B.Cu) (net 2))
 (segment (start 111.76 99.06) (end 111.76 104.14) (width 1) (layer B.Cu) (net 2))
 (segment (start 111.76 104.14) (end 118.11 104.14) (width 1) (layer B.Cu) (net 2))
 (segment (start 123.19 109.22) (end 127 109.22) (width 1) (layer B.Cu) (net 2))
 (segment (start 118.11 104.14) (end 123.19 109.22) (width 1) (layer B.Cu) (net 2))
 (segment (start 111.76 111.76) (end 119.38 111.76) (width 1) (layer B.Cu) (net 4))
 (segment (start 121.92 111.76) (end 127 106.68) (width 1) (layer F.Cu) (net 4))
 (segment (start 119.38 111.76) (end 121.92 111.76) (width 1) (layer F.Cu) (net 4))
 (segment (start 91.03 96.09) (end 91.44 96.5) (width 1) (layer B.Cu) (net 6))
 (segment (start 76.2 96.09) (end 91.03 96.09) (width 1) (layer B.Cu) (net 6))
 (segment (start 91.44 96.5) (end 94 96.5) (width 1) (layer B.Cu) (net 6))
 (segment (start 116.02001 94.79999) (end 119.38 91.44) (width 1) (layer B.Cu) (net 6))
 (segment (start 95.70001 94.79999) (end 116.02001 94.79999) (width 1) (layer B.Cu) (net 6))
 (segment (start 94 96.5) (end 95.70001 94.79999) (width 1) (layer B.Cu) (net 6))
 (segment (start 119.38 91.44) (end 119.38 86.36) (width 1) (layer B.Cu) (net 6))
 (segment (start 121.92 86.36) (end 127 81.28) (width 1) (layer B.Cu) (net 6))
 (segment (start 119.38 86.36) (end 121.92 86.36) (width 1) (layer B.Cu) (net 6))
 (segment (start 127 78.74) (end 119.38 78.74) (width 1) (layer B.Cu) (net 7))
 (segment (start 119.38 78.74) (end 111.76 78.74) (width 1) (layer B.Cu) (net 7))
 (segment (start 88.9 66.04) (end 86.36 63.5) (width 1) (layer B.Cu) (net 3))
 (segment (start 91.44 66.04) (end 88.9 66.04) (width 1) (layer B.Cu) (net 3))
 (segment (start 96.52 60.96) (end 91.44 66.04) (width 1) (layer B.Cu) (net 3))
 (segment (start 73.69999 40.60001) (end 76.2 38.1) (width 1) (layer B.Cu) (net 3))
 (segment (start 73.69999 48.980735) (end 73.69999 40.60001) (width 1) (layer B.Cu) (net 3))
 (segment (start 78.059255 53.34) (end 73.69999 48.980735) (width 1) (layer B.Cu) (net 3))
 (segment (start 81.28 53.34) (end 78.059255 53.34) (width 1) (layer B.Cu) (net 3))
 (segment (start 91.44 63.5) (end 81.28 53.34) (width 1) (layer B.Cu) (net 3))
 (segment (start 91.44 66.04) (end 91.44 63.5) (width 1) (layer B.Cu) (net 3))
 (segment (start 78.74 63.5) (end 86.36 71.12) (width 1) (layer B.Cu) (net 8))
 (segment (start 76.2 63.5) (end 78.74 63.5) (width 1) (layer B.Cu) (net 8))
 (segment (start 88.9 68.58) (end 86.36 71.12) (width 1) (layer B.Cu) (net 8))
 (segment (start 91.44 68.58) (end 88.9 68.58) (width 1) (layer B.Cu) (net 8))
 (segment (start 76.2 121.92) (end 76.2 106.25) (width 1) (layer B.Cu) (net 22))
 (segment (start 98.94 101.54) (end 98.94 115.69) (width 1) (layer F.Cu) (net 20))
 (segment (start 87.63 127) (end 76.2 127) (width 1) (layer F.Cu) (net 20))
 (segment (start 98.94 115.69) (end 87.63 127) (width 1) (layer F.Cu) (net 20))
 (segment (start 83.82 76.2) (end 91.44 76.2) (width 1) (layer B.Cu) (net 21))
 (segment (start 76.2 68.58) (end 83.82 76.2) (width 1) (layer B.Cu) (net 21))
 (segment (start 113.03 123.19) (end 113.03 132.08) (width 1) (layer B.Cu) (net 19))
 (segment (start 142.470001 127.230001) (end 139.7 124.46) (width 1) (layer B.Cu) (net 11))
 (segment (start 142.470001 130.579999) (end 142.470001 127.230001) (width 1) (layer B.Cu) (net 11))
 (segment (start 140.97 132.08) (end 142.470001 130.579999) (width 1) (layer B.Cu) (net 11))
 (segment (start 133.35 129.54) (end 133.35 123.19) (width 1) (layer B.Cu) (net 12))
 (segment (start 111.76 71.12) (end 111.76 67.31) (width 1) (layer B.Cu) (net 16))
 (segment (start 134.389999 59.459999) (end 135.89 60.96) (width 1) (layer B.Cu) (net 16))
 (segment (start 119.610001 59.459999) (end 134.389999 59.459999) (width 1) (layer B.Cu) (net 16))
 (segment (start 111.76 67.31) (end 119.610001 59.459999) (width 1) (layer B.Cu) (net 16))
 (segment (start 92.71 67.31) (end 96.52 71.12) (width 1) (layer B.Cu) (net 9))
 (segment (start 91.44 67.31) (end 92.71 67.31) (width 1) (layer B.Cu) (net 9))
 (segment (start 96.52 71.12) (end 101.6 71.12) (width 1) (layer B.Cu) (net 9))
 (segment (start 134.62 81.28) (end 139.7 81.28) (width 1) (layer B.Cu) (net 15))
 (segment (start 139.7 81.28) (end 139.7 72.39) (width 1) (layer B.Cu) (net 15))
 (segment (start 138.43 71.12) (end 138.43 60.96) (width 1) (layer B.Cu) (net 15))
 (segment (start 139.7 72.39) (end 138.43 71.12) (width 1) (layer B.Cu) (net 15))
 (segment (start 134.62 109.22) (end 139.7 109.22) (width 1) (layer B.Cu) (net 1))
 (segment (start 143.51 63.5) (end 140.97 60.96) (width 1) (layer B.Cu) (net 1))
 (segment (start 143.51 105.41) (end 143.51 63.5) (width 1) (layer B.Cu) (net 1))
 (segment (start 139.7 109.22) (end 143.51 105.41) (width 1) (layer B.Cu) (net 1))
 (segment (start 76.2 132.08) (end 96.52 132.08) (width 1) (layer B.Cu) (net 17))
 (segment (start 101.6 137.16) (end 113.03 137.16) (width 1) (layer B.Cu) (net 17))
 (segment (start 96.52 132.08) (end 101.6 137.16) (width 1) (layer B.Cu) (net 17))
 (segment (start 116.84 137.16) (end 118.11 138.43) (width 1) (layer B.Cu) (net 17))
 (segment (start 113.03 137.16) (end 116.84 137.16) (width 1) (layer B.Cu) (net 17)))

